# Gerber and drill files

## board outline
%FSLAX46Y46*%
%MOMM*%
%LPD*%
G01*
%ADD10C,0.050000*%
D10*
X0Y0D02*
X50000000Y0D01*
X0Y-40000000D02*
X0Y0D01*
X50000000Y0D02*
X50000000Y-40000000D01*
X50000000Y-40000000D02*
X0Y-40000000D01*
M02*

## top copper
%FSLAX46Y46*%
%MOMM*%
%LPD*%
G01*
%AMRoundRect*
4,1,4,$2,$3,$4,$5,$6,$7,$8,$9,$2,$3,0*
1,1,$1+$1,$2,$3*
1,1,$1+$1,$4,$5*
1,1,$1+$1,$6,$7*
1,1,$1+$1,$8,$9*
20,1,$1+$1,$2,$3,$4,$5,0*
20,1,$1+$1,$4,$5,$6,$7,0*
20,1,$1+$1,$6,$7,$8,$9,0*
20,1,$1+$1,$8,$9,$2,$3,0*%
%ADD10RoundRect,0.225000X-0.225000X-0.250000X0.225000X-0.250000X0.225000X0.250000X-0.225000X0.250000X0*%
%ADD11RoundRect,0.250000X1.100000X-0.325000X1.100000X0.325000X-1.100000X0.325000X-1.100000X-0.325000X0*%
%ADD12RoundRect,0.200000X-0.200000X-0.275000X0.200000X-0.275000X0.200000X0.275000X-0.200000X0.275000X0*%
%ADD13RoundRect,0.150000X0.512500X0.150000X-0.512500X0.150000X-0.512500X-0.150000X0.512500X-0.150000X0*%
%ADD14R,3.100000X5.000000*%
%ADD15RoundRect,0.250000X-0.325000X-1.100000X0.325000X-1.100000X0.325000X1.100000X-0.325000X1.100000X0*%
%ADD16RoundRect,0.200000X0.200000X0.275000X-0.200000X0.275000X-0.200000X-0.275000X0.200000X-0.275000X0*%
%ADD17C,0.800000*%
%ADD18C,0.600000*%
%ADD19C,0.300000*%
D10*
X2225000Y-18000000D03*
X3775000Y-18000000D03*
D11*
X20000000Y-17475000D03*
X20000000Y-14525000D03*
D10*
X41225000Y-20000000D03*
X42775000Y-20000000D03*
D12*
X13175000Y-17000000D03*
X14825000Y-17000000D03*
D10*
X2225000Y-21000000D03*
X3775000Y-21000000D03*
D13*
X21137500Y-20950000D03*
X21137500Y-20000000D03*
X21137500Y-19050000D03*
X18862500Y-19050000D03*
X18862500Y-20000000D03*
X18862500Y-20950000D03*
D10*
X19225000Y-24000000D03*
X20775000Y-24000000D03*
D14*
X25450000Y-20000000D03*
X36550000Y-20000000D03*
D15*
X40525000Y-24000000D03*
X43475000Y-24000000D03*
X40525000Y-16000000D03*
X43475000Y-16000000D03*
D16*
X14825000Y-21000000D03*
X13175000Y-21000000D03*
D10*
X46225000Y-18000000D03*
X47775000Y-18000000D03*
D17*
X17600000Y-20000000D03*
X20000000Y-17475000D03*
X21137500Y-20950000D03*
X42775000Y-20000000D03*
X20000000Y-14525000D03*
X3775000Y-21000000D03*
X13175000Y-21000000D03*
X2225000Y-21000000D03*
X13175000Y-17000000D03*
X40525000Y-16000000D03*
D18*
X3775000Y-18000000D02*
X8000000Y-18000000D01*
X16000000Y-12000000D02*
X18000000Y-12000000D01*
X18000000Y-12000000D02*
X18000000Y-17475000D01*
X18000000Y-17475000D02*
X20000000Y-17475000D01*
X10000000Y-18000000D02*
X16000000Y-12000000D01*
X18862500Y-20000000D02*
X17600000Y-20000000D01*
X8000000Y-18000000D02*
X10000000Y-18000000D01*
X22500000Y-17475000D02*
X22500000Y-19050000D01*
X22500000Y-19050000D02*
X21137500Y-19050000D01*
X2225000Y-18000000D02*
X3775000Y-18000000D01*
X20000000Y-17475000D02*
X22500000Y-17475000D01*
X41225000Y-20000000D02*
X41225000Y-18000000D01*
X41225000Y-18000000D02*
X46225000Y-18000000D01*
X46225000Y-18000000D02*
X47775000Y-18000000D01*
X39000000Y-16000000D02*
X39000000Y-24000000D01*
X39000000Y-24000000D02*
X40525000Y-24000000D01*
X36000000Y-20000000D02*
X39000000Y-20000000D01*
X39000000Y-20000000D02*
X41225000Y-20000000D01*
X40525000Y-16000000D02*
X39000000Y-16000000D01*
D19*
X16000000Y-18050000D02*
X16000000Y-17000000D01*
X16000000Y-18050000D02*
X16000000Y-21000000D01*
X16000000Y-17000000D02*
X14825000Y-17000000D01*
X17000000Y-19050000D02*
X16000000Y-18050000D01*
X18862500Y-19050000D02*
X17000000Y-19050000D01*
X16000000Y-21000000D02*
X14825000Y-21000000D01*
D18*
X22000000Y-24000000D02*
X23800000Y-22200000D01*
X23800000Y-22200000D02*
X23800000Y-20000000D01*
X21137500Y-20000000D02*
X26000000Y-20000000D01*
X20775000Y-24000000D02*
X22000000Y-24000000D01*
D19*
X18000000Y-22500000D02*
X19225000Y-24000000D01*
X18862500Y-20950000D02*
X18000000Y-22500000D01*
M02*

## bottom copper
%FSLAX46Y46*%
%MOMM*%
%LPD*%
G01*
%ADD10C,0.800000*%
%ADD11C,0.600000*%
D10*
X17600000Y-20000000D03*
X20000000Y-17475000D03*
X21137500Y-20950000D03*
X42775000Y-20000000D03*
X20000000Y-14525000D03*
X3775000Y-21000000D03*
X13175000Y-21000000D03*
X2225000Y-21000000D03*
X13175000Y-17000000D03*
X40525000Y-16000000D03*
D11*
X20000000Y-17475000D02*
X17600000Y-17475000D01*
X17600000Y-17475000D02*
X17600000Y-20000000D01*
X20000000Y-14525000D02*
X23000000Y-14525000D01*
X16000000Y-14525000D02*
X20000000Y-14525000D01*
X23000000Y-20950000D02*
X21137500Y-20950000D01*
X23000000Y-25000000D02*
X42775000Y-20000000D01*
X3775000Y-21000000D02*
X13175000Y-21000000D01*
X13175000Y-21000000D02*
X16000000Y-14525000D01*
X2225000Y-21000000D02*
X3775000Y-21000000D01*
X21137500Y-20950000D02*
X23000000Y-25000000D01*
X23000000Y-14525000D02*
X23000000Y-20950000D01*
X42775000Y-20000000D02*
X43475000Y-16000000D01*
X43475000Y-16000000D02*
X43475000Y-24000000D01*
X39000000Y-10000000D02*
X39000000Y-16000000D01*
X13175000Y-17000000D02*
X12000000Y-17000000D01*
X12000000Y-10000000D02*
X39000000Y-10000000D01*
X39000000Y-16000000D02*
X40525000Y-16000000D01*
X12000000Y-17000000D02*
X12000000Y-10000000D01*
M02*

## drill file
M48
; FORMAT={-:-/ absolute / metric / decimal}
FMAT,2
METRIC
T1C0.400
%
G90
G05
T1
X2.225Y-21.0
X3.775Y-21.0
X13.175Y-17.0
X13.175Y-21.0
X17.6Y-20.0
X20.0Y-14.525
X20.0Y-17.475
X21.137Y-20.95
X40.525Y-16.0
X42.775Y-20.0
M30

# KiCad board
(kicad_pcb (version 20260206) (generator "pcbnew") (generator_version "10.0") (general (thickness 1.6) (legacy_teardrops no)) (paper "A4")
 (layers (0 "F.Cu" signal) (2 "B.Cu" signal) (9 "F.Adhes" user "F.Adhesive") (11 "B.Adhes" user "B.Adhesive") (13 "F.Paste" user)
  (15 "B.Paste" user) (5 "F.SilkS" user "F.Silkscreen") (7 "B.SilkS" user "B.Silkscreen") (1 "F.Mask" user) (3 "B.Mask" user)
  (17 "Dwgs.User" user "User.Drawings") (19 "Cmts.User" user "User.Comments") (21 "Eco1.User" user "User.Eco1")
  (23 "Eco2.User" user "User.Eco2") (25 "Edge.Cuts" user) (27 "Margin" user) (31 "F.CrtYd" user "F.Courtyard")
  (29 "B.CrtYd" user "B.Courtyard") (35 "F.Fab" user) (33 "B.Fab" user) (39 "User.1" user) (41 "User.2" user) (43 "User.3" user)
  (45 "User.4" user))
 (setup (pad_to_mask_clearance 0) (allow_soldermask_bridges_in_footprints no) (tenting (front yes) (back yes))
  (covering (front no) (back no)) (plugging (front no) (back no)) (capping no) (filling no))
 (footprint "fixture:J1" (layer "F.Cu") (at 3 18)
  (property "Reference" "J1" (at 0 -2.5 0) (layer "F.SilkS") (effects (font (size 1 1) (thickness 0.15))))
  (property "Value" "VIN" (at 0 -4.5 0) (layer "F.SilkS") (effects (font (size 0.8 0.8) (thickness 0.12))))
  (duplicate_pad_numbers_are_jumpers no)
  (pad "1" smd roundrect (at -0.775 0) (size 0.9 0.95) (layers "F.Cu" "F.Mask" "F.Paste") (roundrect_rratio 0.25) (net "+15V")
   (thermal_bridge_angle 45))
  (pad "2" smd roundrect (at 0.775 0) (size 0.9 0.95) (layers "F.Cu" "F.Mask" "F.Paste") (roundrect_rratio 0.25) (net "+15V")
   (thermal_bridge_angle 45)))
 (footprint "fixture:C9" (layer "F.Cu") (at 20 16 90)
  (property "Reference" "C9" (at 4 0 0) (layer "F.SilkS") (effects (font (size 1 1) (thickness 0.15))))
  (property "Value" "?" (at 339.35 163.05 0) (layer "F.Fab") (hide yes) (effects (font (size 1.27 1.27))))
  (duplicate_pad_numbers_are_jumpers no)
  (pad "1" smd roundrect (at -1.475 0 90) (size 1.15 2.7) (layers "F.Cu" "F.Mask" "F.Paste") (roundrect_rratio 0.217391) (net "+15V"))
  (pad "2" smd roundrect (at 1.475 0 90) (size 1.15 2.7) (layers "F.Cu" "F.Mask" "F.Paste") (roundrect_rratio 0.217391) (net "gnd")))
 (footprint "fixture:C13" (layer "F.Cu") (at 42 20)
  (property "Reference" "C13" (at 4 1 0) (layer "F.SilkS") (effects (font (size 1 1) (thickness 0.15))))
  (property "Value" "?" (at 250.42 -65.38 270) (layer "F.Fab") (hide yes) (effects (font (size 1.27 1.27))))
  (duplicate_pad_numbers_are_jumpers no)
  (pad "1" smd roundrect (at -0.775 0) (size 0.9 0.95) (layers "F.Cu" "F.Mask" "F.Paste") (roundrect_rratio 0.25) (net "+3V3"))
  (pad "2" smd roundrect (at 0.775 0) (size 0.9 0.95) (layers "F.Cu" "F.Mask" "F.Paste") (roundrect_rratio 0.25) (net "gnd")))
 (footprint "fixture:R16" (layer "F.Cu") (at 14 17)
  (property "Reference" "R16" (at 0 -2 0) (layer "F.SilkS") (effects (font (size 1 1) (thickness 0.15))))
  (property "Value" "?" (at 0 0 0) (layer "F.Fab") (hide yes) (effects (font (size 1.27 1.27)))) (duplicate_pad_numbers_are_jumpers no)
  (pad "1" smd roundrect (at -0.825 0) (size 0.8 0.95) (layers "F.Cu" "F.Mask" "F.Paste") (roundrect_rratio 0.25) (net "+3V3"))
  (pad "2" smd roundrect (at 0.825 0) (size 0.8 0.95) (layers "F.Cu" "F.Mask" "F.Paste") (roundrect_rratio 0.25) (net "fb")))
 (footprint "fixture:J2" (layer "F.Cu") (at 3 21)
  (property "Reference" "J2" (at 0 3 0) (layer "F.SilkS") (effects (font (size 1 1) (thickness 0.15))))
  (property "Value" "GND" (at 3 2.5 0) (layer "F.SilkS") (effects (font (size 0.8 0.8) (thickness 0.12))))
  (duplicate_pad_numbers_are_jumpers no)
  (pad "1" smd roundrect (at -0.775 0) (size 0.9 0.95) (layers "F.Cu" "F.Mask" "F.Paste") (roundrect_rratio 0.25) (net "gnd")
   (thermal_bridge_angle 45))
  (pad "2" smd roundrect (at 0.775 0) (size 0.9 0.95) (layers "F.Cu" "F.Mask" "F.Paste") (roundrect_rratio 0.25) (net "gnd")
   (thermal_bridge_angle 45)))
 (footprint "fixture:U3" (layer "F.Cu") (at 20 20 180)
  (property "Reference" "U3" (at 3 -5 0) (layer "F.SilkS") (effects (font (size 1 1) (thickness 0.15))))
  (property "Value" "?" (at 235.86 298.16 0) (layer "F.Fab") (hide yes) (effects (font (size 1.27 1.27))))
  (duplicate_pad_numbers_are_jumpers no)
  (pad "1" smd roundrect (at -1.1375 -0.95 180) (size 1.325 0.6) (layers "F.Cu" "F.Mask" "F.Paste") (roundrect_rratio 0.25) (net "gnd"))
  (pad "2" smd roundrect (at -1.1375 0 180) (size 1.325 0.6) (layers "F.Cu" "F.Mask" "F.Paste") (roundrect_rratio 0.25) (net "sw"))
  (pad "3" smd roundrect (at -1.1375 0.95 180) (size 1.325 0.6) (layers "F.Cu" "F.Mask" "F.Paste") (roundrect_rratio 0.25) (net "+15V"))
  (pad "4" smd roundrect (at 1.1375 0.95 180) (size 1.325 0.6) (layers "F.Cu" "F.Mask" "F.Paste") (roundrect_rratio 0.25) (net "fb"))
  (pad "5" smd roundrect (at 1.1375 0 180) (size 1.325 0.6) (layers "F.Cu" "F.Mask" "F.Paste") (roundrect_rratio 0.25) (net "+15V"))
  (pad "6" smd roundrect (at 1.1375 -0.95 180) (size 1.325 0.6) (layers "F.Cu" "F.Mask" "F.Paste") (roundrect_rratio 0.25) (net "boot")))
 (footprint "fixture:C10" (layer "F.Cu") (at 20 24)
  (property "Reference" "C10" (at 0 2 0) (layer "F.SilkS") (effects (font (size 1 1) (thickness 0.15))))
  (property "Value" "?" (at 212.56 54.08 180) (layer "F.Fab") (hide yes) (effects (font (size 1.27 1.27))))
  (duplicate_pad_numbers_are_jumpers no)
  (pad "1" smd roundrect (at -0.775 0) (size 0.9 0.95) (layers "F.Cu" "F.Mask" "F.Paste") (roundrect_rratio 0.25) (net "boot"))
  (pad "2" smd roundrect (at 0.775 0) (size 0.9 0.95) (layers "F.Cu" "F.Mask" "F.Paste") (roundrect_rratio 0.25) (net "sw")))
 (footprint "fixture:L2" (layer "F.Cu") (at 31 20)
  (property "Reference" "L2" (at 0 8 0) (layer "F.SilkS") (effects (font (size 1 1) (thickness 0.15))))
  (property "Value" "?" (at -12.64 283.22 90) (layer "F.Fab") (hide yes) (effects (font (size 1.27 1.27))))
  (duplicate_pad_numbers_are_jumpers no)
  (pad "1" smd rect (at -5.55 0) (size 3.1 5) (layers "F.Cu" "F.Mask" "F.Paste") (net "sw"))
  (pad "2" smd rect (at 5.55 0) (size 3.1 5) (layers "F.Cu" "F.Mask" "F.Paste") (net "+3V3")))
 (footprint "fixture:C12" (layer "F.Cu") (at 42 24)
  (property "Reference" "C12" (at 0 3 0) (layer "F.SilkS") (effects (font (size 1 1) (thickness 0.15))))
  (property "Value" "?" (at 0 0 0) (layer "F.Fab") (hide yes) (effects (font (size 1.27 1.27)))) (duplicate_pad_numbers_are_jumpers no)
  (pad "1" smd roundrect (at -1.475 0) (size 1.15 2.7) (layers "F.Cu" "F.Mask" "F.Paste") (roundrect_rratio 0.217391) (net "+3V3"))
  (pad "2" smd roundrect (at 1.475 0) (size 1.15 2.7) (layers "F.Cu" "F.Mask" "F.Paste") (roundrect_rratio 0.217391) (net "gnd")))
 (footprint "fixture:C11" (layer "F.Cu") (at 42 16)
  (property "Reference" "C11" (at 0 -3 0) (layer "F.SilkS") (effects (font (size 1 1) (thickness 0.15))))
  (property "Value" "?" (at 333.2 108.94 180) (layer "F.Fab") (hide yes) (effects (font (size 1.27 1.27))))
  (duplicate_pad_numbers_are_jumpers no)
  (pad "1" smd roundrect (at -1.475 0) (size 1.15 2.7) (layers "F.Cu" "F.Mask" "F.Paste") (roundrect_rratio 0.217391) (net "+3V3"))
  (pad "2" smd roundrect (at 1.475 0) (size 1.15 2.7) (layers "F.Cu" "F.Mask" "F.Paste") (roundrect_rratio 0.217391) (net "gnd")))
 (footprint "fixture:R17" (layer "F.Cu") (at 14 21 180)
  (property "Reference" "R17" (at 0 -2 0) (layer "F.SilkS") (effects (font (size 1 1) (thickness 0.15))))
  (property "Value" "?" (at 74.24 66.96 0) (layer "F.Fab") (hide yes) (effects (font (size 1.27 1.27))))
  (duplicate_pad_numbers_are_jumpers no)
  (pad "1" smd roundrect (at -0.825 0 180) (size 0.8 0.95) (layers "F.Cu" "F.Mask" "F.Paste") (roundrect_rratio 0.25) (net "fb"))
  (pad "2" smd roundrect (at 0.825 0 180) (size 0.8 0.95) (layers "F.Cu" "F.Mask" "F.Paste") (roundrect_rratio 0.25) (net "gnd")))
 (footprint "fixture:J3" (layer "F.Cu") (at 47 18)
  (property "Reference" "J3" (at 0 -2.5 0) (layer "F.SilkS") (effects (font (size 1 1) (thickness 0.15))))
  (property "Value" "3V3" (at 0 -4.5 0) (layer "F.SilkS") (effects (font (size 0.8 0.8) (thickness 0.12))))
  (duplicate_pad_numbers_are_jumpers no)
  (pad "1" smd roundrect (at -0.775 0) (size 0.9 0.95) (layers "F.Cu" "F.Mask" "F.Paste") (roundrect_rratio 0.25) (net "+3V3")
   (thermal_bridge_angle 45))
  (pad "2" smd roundrect (at 0.775 0) (size 0.9 0.95) (layers "F.Cu" "F.Mask" "F.Paste") (roundrect_rratio 0.25) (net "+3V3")
   (thermal_bridge_angle 45)))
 (gr_line (start 0 0) (end 50 0) (stroke (width 0.05) (type default)) (layer "Edge.Cuts"))
 (gr_line (start 0 40) (end 0 0) (stroke (width 0.05) (type default)) (layer "Edge.Cuts"))
 (gr_line (start 50 0) (end 50 40) (stroke (width 0.05) (type default)) (layer "Edge.Cuts"))
 (gr_line (start 50 40) (end 0 40) (stroke (width 0.05) (type default)) (layer "Edge.Cuts"))
 (segment (start 3.775 18) (end 8 18) (width 0.6) (layer "F.Cu") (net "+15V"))
 (segment (start 16 12) (end 18 12) (width 0.6) (layer "F.Cu") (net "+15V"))
 (segment (start 18 12) (end 18 17.475) (width 0.6) (layer "F.Cu") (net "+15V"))
 (segment (start 18 17.475) (end 20 17.475) (width 0.6) (layer "F.Cu") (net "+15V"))
 (segment (start 10 18) (end 16 12) (width 0.6) (layer "F.Cu") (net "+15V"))
 (segment (start 18.8625 20) (end 17.6 20) (width 0.6) (layer "F.Cu") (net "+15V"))
 (segment (start 8 18) (end 10 18) (width 0.6) (layer "F.Cu") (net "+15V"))
 (segment (start 22.5 17.475) (end 22.5 19.05) (width 0.6) (layer "F.Cu") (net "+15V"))
 (segment (start 22.5 19.05) (end 21.1375 19.05) (width 0.6) (layer "F.Cu") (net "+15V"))
 (segment (start 2.225 18) (end 3.775 18) (width 0.6) (layer "F.Cu") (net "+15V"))
 (segment (start 20 17.475) (end 22.5 17.475) (width 0.6) (layer "F.Cu") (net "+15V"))
 (via (at 17.6 20) (size 0.8) (drill 0.4) (layers "F.Cu" "B.Cu") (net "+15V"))
 (via (at 20 17.475) (size 0.8) (drill 0.4) (layers "F.Cu" "B.Cu") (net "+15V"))
 (segment (start 20 17.475) (end 17.6 17.475) (width 0.6) (layer "B.Cu") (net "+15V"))
 (segment (start 17.6 17.475) (end 17.6 20) (width 0.6) (layer "B.Cu") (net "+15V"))
 (via (at 21.1375 20.95) (size 0.8) (drill 0.4) (layers "F.Cu" "B.Cu") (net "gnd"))
 (via (at 42.775 20) (size 0.8) (drill 0.4) (layers "F.Cu" "B.Cu") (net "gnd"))
 (via (at 20 14.525) (size 0.8) (drill 0.4) (layers "F.Cu" "B.Cu") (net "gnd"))
 (via (at 3.775 21) (size 0.8) (drill 0.4) (layers "F.Cu" "B.Cu") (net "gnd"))
 (via (at 13.175 21) (size 0.8) (drill 0.4) (layers "F.Cu" "B.Cu") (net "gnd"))
 (via (at 2.225 21) (size 0.8) (drill 0.4) (layers "F.Cu" "B.Cu") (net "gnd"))
 (segment (start 20 14.525) (end 23 14.525) (width 0.6) (layer "B.Cu") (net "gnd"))
 (segment (start 16 14.525) (end 20 14.525) (width 0.6) (layer "B.Cu") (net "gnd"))
 (segment (start 23 20.95) (end 21.1375 20.95) (width 0.6) (layer "B.Cu") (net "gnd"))
 (segment (start 23 25) (end 42.775 20) (width 0.6) (layer "B.Cu") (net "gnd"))
 (segment (start 3.775 21) (end 13.175 21) (width 0.6) (layer "B.Cu") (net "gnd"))
 (segment (start 13.175 21) (end 16 14.525) (width 0.6) (layer "B.Cu") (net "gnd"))
 (segment (start 2.225 21) (end 3.775 21) (width 0.6) (layer "B.Cu") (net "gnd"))
 (segment (start 21.1375 20.95) (end 23 25) (width 0.6) (layer "B.Cu") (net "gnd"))
 (segment (start 23 14.525) (end 23 20.95) (width 0.6) (layer "B.Cu") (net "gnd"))
 (segment (start 42.775 20) (end 43.475 16) (width 0.6) (layer "B.Cu") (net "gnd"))
 (segment (start 43.475 16) (end 43.475 24) (width 0.6) (layer "B.Cu") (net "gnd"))
 (segment (start 41.225 20) (end 41.225 18) (width 0.6) (layer "F.Cu") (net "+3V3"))
 (segment (start 41.225 18) (end 46.225 18) (width 0.6) (layer "F.Cu") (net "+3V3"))
 (segment (start 46.225 18) (end 47.775 18) (width 0.6) (layer "F.Cu") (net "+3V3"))
 (segment (start 39 16) (end 39 24) (width 0.6) (layer "F.Cu") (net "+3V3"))
 (segment (start 39 24) (end 40.525 24) (width 0.6) (layer "F.Cu") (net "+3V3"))
 (segment (start 36 20) (end 39 20) (width 0.6) (layer "F.Cu") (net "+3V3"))
 (segment (start 39 20) (end 41.225 20) (width 0.6) (layer "F.Cu") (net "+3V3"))
 (segment (start 40.525 16) (end 39 16) (width 0.6) (layer "F.Cu") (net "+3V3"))
 (via (at 13.175 17) (size 0.8) (drill 0.4) (layers "F.Cu" "B.Cu") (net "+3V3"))
 (via (at 40.525 16) (size 0.8) (drill 0.4) (layers "F.Cu" "B.Cu") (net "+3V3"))
 (segment (start 39 10) (end 39 16) (width 0.6) (layer "B.Cu") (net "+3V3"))
 (segment (start 13.175 17) (end 12 17) (width 0.6) (layer "B.Cu") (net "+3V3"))
 (segment (start 12 10) (end 39 10) (width 0.6) (layer "B.Cu") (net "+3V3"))
 (segment (start 39 16) (end 40.525 16) (width 0.6) (layer "B.Cu") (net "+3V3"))
 (segment (start 12 17) (end 12 10) (width 0.6) (layer "B.Cu") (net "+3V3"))
 (segment (start 16 18.05) (end 16 17) (width 0.3) (layer "F.Cu") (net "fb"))
 (segment (start 16 18.05) (end 16 21) (width 0.3) (layer "F.Cu") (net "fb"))
 (segment (start 16 17) (end 14.825 17) (width 0.3) (layer "F.Cu") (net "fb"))
 (segment (start 17 19.05) (end 16 18.05) (width 0.3) (layer "F.Cu") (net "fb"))
 (segment (start 18.8625 19.05) (end 17 19.05) (width 0.3) (layer "F.Cu") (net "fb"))
 (segment (start 16 21) (end 14.825 21) (width 0.3) (layer "F.Cu") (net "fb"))
 (segment (start 22 24) (end 23.8 22.2) (width 0.6) (layer "F.Cu") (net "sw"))
 (segment (start 23.8 22.2) (end 23.8 20) (width 0.6) (layer "F.Cu") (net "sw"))
 (segment (start 21.1375 20) (end 26 20) (width 0.6) (layer "F.Cu") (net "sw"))
 (segment (start 20.775 24) (end 22 24) (width 0.6) (layer "F.Cu") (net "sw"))
 (segment (start 18 22.5) (end 19.225 24) (width 0.3) (layer "F.Cu") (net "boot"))
 (segment (start 18.8625 20.95) (end 18 22.5) (width 0.3) (layer "F.Cu") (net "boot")))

